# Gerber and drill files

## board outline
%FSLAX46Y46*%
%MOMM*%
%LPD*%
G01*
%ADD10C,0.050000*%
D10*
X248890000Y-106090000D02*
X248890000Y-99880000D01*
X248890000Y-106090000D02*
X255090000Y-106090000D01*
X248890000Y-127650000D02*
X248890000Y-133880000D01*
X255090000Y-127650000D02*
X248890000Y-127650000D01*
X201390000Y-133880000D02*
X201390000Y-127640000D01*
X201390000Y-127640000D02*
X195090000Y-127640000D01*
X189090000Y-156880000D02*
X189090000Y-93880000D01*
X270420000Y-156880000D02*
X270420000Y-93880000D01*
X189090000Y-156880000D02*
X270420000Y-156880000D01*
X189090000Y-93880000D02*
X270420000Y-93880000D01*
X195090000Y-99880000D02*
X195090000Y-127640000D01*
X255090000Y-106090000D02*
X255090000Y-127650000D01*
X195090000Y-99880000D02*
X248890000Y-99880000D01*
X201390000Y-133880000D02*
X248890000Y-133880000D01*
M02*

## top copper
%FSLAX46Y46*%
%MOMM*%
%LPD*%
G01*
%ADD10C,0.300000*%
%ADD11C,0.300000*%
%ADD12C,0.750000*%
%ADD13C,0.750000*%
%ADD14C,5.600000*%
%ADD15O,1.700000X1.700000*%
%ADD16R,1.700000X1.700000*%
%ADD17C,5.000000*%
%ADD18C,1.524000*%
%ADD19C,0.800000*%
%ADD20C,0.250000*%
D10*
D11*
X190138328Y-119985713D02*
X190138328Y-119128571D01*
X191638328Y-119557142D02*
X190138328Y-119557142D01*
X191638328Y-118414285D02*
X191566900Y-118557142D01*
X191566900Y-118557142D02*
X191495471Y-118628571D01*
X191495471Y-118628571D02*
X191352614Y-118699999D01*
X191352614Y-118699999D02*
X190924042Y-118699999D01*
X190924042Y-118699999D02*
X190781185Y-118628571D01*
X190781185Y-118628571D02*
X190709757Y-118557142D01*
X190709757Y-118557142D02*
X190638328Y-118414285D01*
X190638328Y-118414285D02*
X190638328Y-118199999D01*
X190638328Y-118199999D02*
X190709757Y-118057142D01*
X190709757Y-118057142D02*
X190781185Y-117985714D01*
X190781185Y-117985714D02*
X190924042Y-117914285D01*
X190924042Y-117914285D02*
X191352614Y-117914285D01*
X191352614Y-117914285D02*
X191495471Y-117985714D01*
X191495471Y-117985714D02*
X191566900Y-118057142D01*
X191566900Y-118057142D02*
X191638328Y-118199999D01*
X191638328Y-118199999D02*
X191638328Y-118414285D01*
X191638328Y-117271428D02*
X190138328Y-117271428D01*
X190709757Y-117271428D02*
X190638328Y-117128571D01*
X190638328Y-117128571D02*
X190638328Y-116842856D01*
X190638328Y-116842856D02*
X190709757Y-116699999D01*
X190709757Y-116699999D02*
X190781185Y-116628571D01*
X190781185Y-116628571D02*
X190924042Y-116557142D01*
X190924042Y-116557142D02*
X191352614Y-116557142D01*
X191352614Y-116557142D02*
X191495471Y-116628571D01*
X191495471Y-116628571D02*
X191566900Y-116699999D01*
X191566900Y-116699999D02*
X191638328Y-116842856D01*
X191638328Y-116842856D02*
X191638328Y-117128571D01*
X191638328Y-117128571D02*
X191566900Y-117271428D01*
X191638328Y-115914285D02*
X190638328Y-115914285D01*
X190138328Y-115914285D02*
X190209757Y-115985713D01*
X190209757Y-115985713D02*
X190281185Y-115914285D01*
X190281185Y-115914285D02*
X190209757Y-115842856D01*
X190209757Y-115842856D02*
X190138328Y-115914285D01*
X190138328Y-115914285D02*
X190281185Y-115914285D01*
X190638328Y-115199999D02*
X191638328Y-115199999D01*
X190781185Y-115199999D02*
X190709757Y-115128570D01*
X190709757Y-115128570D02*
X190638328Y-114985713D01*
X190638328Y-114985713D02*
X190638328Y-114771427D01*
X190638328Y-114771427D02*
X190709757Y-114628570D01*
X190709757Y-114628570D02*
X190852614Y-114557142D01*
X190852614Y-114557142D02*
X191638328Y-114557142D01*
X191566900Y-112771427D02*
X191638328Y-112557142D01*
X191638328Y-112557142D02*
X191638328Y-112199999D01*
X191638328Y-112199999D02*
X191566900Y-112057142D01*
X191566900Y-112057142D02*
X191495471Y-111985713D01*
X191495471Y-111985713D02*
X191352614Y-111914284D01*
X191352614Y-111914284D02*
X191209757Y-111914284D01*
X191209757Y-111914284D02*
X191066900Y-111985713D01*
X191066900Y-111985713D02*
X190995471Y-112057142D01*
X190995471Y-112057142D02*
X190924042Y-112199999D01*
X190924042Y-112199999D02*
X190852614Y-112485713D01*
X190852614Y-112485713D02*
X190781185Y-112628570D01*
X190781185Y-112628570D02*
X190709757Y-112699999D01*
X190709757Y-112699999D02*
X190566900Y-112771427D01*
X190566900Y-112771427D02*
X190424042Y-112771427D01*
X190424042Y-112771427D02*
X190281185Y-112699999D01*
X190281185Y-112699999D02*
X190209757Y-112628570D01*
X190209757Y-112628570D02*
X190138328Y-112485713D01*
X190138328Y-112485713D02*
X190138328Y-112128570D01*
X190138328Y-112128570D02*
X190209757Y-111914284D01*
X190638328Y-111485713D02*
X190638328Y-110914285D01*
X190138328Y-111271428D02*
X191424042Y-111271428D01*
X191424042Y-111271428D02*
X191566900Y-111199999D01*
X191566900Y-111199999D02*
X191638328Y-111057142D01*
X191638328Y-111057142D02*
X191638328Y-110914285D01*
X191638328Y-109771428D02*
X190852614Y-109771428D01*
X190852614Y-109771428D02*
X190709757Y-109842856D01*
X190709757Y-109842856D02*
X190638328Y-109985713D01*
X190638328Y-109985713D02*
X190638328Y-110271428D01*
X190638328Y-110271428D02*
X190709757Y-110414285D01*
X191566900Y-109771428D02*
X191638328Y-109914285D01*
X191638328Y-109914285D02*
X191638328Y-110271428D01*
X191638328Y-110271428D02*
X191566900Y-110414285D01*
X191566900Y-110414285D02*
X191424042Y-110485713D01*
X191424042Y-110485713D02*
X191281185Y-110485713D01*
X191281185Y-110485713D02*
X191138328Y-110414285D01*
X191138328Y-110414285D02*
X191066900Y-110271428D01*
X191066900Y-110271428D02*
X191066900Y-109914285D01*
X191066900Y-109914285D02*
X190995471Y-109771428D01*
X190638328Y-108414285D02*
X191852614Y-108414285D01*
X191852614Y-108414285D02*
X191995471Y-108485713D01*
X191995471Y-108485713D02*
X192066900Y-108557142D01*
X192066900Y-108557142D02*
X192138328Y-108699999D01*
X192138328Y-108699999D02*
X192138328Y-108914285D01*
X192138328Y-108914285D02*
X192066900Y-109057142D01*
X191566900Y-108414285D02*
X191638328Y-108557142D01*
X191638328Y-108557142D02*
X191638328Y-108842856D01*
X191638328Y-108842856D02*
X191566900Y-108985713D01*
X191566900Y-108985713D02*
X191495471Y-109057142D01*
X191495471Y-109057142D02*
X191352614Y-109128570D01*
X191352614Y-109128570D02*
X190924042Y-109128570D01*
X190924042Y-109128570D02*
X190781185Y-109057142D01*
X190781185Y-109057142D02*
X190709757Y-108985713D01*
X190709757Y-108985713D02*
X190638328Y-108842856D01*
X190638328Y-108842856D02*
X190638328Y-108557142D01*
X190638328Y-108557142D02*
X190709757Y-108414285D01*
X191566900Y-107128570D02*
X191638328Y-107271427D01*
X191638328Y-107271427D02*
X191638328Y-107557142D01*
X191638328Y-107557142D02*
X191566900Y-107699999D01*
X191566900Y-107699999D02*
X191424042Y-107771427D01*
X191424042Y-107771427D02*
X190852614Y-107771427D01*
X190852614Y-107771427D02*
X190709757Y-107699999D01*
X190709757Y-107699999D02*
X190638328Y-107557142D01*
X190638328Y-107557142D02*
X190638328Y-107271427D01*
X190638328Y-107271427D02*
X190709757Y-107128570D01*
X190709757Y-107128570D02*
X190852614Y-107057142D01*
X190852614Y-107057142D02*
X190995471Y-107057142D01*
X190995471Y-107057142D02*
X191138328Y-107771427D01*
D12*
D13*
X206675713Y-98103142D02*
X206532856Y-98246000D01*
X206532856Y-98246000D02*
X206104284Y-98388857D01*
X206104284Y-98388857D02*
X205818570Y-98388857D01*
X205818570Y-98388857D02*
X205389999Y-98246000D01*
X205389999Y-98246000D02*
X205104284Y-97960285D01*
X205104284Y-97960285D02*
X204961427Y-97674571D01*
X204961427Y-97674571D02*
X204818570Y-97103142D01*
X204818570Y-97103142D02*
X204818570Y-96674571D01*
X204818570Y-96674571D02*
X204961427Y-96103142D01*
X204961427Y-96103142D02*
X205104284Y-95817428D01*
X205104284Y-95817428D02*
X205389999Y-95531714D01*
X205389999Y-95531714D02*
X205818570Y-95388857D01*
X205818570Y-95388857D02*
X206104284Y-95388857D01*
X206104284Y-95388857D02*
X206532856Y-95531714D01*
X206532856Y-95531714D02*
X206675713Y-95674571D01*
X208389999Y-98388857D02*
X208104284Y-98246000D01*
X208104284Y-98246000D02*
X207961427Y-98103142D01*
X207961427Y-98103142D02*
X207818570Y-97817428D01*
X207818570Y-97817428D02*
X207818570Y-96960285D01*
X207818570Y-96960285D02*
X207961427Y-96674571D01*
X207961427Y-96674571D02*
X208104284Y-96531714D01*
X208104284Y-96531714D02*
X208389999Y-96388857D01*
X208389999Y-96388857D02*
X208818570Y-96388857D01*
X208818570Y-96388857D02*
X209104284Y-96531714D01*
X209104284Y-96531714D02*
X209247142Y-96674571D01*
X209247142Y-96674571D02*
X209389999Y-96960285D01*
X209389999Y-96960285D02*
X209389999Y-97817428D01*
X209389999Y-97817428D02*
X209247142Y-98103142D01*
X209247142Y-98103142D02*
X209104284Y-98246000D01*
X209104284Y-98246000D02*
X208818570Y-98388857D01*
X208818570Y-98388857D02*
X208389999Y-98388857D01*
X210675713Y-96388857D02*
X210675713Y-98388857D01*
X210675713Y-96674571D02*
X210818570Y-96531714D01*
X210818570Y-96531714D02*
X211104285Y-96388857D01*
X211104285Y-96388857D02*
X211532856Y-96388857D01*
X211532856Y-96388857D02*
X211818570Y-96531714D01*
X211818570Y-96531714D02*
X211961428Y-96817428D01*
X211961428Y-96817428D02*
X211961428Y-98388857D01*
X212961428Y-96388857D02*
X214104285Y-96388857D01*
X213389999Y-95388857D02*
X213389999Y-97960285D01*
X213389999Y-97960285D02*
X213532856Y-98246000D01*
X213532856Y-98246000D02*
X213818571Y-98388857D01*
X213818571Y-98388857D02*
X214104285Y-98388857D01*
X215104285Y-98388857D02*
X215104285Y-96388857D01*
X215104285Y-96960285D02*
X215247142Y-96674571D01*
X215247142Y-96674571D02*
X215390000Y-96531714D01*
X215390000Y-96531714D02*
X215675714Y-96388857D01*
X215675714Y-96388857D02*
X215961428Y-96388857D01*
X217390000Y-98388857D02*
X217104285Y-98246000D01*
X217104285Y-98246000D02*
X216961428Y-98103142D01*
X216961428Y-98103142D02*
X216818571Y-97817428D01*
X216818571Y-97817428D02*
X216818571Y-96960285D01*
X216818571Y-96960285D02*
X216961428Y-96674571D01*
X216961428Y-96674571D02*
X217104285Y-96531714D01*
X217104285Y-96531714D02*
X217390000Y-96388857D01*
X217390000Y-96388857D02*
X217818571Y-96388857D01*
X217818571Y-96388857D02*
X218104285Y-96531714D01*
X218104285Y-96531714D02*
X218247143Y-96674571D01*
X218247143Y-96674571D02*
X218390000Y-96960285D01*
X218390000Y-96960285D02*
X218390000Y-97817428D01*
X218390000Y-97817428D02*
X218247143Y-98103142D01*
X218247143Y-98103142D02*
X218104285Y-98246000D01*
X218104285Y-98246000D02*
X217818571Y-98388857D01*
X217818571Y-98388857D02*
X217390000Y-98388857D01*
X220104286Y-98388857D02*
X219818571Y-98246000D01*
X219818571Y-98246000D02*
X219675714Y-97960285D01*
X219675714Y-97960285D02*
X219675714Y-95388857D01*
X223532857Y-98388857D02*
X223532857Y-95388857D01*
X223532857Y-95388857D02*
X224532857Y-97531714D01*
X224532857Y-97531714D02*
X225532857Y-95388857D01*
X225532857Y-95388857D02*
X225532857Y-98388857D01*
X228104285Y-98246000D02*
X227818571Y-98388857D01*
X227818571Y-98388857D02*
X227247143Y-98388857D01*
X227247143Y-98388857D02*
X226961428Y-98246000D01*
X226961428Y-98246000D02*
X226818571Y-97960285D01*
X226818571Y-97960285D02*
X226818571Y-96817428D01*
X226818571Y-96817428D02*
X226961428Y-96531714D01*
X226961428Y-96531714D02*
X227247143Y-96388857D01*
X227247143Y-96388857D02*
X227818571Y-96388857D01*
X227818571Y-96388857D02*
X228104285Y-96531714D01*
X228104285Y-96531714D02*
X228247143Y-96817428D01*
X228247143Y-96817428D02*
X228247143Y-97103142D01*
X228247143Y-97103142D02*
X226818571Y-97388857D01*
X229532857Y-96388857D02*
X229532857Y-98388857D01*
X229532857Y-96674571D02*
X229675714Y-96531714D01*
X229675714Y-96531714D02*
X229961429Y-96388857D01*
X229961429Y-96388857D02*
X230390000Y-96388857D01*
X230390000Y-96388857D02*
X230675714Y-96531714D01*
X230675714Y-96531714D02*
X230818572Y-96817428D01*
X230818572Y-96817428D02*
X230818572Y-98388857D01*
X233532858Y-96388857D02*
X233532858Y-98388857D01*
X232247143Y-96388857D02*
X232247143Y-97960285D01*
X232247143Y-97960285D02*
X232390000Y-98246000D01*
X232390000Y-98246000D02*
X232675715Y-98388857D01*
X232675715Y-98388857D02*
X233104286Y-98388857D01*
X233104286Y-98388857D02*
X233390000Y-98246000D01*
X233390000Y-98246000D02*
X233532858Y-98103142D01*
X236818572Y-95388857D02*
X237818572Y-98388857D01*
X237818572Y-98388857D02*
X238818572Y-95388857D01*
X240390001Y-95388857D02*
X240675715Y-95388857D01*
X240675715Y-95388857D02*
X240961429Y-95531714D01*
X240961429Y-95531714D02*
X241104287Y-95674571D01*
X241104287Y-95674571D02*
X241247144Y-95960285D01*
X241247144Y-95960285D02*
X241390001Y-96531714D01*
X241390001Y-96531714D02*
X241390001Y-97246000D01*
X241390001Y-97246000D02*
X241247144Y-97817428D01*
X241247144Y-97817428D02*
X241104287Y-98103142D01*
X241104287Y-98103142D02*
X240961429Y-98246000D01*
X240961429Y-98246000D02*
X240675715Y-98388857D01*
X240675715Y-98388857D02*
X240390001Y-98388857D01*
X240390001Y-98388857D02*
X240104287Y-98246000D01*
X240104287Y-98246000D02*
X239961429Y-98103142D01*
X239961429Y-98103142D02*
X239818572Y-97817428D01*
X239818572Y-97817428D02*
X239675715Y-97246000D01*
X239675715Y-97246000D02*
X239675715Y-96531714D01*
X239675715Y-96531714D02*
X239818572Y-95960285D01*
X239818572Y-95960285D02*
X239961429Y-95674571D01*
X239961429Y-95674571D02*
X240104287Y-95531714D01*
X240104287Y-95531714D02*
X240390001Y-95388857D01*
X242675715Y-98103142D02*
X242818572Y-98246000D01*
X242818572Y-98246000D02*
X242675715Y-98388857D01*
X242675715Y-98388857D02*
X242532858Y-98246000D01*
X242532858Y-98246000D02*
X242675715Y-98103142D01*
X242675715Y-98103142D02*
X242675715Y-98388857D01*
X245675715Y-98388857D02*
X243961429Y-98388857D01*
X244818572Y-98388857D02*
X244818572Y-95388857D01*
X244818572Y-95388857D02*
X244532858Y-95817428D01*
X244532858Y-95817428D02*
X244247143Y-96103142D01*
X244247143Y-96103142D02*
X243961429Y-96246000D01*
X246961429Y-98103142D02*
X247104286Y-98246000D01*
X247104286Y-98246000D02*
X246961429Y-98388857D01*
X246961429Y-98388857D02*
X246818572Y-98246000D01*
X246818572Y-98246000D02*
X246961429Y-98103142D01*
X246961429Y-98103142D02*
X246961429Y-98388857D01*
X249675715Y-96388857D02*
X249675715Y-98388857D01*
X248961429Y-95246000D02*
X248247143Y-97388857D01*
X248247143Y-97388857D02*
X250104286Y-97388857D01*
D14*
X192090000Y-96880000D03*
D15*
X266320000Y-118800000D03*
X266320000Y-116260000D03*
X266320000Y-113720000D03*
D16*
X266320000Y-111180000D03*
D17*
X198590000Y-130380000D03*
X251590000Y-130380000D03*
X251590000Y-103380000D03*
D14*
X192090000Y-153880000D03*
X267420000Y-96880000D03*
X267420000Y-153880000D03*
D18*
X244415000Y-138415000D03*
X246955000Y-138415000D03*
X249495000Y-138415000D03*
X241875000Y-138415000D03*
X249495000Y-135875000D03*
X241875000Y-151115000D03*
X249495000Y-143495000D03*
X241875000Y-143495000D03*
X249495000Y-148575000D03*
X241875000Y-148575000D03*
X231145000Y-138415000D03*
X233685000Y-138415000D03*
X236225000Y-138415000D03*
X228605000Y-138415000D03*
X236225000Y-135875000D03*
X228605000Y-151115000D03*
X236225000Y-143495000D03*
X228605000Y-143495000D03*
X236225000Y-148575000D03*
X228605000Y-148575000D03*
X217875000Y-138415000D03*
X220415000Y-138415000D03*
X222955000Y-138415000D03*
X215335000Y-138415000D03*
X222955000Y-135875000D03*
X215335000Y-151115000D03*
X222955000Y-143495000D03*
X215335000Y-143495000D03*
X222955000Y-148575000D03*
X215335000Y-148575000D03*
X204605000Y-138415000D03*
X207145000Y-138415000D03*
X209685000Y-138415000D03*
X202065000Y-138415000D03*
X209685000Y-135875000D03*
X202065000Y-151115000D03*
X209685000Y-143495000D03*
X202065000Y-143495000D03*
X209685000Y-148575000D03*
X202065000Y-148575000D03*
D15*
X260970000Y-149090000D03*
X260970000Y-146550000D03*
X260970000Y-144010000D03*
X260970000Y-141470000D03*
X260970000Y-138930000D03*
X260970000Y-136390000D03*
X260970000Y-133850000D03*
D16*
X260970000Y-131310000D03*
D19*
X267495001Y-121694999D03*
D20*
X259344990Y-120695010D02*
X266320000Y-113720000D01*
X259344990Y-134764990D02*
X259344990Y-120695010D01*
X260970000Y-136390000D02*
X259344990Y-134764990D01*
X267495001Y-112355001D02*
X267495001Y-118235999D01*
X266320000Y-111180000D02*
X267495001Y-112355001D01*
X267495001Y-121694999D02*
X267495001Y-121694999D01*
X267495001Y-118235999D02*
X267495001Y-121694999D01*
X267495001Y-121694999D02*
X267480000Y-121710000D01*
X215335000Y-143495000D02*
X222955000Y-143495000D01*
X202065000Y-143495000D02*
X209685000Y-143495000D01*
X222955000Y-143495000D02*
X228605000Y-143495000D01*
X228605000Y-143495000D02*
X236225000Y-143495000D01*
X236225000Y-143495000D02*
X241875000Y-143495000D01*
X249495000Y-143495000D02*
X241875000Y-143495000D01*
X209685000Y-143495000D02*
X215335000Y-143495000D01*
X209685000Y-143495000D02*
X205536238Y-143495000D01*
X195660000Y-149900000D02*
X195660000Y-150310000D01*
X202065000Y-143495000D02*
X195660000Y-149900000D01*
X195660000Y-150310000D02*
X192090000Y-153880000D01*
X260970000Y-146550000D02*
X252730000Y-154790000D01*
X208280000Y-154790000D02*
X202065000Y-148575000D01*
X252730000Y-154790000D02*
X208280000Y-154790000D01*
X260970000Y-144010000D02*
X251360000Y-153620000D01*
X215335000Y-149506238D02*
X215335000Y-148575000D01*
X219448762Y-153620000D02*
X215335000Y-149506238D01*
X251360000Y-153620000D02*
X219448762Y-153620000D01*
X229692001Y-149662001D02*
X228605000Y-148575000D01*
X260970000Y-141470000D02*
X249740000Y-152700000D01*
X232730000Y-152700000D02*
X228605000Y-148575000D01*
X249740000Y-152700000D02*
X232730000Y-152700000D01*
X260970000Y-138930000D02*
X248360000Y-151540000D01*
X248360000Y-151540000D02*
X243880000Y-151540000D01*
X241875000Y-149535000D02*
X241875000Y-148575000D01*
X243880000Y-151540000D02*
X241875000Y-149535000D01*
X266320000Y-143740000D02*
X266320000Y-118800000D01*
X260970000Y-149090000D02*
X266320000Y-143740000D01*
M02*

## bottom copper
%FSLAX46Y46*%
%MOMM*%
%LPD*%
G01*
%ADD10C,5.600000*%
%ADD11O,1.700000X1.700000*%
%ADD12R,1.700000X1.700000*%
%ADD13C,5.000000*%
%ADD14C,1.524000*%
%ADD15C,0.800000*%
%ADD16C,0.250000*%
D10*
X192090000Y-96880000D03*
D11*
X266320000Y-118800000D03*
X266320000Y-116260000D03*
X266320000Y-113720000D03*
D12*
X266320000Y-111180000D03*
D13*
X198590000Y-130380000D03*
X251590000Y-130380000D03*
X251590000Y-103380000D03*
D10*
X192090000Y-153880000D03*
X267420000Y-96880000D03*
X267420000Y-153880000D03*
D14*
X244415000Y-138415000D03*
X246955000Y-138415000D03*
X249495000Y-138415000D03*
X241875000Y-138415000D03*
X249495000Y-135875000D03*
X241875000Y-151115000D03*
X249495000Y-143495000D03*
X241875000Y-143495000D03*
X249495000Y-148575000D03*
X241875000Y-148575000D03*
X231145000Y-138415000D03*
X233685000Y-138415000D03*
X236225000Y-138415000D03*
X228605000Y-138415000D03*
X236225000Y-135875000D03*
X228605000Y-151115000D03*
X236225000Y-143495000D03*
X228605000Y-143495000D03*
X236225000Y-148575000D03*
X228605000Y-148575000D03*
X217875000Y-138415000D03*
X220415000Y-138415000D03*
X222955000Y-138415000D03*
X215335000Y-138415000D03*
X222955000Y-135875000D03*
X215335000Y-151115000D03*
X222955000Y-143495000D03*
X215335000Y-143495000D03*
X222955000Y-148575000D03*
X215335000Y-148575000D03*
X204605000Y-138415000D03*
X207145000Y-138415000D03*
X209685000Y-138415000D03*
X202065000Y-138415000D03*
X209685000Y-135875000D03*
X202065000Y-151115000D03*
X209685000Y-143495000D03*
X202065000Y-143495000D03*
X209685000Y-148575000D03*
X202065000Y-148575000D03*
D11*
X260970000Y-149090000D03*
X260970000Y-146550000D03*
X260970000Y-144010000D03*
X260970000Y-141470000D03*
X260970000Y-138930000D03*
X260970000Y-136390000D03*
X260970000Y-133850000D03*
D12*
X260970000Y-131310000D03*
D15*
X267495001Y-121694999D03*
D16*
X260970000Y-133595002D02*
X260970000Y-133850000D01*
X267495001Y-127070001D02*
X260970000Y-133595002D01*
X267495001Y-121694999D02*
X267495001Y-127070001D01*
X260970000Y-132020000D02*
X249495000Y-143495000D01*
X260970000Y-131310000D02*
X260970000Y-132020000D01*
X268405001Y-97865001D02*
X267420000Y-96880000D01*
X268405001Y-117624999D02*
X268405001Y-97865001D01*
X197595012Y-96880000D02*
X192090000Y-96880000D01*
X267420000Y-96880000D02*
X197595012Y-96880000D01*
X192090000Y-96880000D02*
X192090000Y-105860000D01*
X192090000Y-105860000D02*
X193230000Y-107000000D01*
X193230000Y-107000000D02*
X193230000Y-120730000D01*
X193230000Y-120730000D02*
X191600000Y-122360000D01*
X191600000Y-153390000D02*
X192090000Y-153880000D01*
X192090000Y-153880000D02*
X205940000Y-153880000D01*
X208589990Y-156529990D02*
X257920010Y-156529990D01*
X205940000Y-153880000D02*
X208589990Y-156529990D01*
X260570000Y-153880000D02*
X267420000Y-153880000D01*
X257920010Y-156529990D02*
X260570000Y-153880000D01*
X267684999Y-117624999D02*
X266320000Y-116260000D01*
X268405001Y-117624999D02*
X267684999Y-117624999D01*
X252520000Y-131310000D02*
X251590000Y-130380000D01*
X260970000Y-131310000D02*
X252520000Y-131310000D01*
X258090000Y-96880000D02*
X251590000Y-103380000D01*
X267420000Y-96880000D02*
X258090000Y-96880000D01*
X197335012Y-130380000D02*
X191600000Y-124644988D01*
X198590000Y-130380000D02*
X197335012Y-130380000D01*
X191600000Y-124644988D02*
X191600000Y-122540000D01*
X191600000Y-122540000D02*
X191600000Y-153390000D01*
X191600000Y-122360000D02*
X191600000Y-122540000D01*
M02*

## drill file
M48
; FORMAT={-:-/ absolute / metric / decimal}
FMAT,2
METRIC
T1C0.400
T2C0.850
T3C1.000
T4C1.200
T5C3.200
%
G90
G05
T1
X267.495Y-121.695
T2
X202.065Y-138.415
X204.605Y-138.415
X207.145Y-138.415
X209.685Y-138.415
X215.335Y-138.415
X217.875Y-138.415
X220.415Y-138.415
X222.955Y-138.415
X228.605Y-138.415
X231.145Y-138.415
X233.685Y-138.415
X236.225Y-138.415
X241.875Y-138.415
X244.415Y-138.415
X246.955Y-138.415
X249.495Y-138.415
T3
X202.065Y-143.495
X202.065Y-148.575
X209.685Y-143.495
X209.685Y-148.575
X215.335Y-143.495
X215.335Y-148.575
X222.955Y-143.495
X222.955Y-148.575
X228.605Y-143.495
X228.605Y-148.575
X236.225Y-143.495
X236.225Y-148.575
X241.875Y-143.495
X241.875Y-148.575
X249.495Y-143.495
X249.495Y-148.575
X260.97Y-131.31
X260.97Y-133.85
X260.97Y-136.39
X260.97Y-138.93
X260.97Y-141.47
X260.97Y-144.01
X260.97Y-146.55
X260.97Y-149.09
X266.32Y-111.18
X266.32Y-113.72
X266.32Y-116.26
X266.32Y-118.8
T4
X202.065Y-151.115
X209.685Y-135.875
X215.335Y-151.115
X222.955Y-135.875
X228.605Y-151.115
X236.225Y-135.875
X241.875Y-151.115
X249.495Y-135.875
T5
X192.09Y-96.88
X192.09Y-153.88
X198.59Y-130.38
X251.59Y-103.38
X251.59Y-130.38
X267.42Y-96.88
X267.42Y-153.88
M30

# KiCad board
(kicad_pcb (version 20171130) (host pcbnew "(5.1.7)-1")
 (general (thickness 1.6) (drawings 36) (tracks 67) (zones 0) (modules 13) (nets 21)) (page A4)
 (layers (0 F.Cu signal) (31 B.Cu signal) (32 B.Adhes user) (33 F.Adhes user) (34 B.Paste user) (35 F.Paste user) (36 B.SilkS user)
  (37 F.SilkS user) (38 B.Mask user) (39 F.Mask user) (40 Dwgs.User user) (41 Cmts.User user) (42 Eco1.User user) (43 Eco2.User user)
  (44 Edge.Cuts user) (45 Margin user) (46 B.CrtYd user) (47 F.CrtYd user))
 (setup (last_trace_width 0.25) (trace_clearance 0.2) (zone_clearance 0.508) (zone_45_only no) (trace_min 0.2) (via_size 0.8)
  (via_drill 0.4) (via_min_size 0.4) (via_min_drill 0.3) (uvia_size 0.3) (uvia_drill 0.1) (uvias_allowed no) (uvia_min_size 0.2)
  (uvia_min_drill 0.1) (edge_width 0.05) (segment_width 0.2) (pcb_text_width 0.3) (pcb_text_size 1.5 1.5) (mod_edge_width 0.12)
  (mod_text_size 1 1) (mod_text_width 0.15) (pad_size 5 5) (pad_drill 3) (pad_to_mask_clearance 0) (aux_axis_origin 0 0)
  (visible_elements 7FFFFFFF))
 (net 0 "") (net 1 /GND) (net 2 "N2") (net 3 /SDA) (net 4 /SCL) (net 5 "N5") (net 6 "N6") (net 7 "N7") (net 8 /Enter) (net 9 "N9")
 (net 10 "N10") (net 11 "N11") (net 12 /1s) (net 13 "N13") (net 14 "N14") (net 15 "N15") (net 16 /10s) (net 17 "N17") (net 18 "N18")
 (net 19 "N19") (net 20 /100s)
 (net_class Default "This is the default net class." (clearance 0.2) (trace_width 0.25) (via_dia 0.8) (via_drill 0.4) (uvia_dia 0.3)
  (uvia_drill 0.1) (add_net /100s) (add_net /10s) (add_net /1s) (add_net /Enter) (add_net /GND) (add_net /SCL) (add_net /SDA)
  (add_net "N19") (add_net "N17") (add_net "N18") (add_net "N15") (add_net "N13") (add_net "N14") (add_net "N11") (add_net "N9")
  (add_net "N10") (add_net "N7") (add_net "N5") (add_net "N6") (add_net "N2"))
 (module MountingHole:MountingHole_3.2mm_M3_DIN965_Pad (layer F.Cu) (at 192.09 96.88)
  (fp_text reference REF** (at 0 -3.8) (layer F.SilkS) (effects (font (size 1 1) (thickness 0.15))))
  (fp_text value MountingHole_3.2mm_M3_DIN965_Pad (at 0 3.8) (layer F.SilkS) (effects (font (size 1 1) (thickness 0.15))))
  (pad 1 thru_hole circle (at 0 0) (size 5.6 5.6) (drill 3.2) (layers *.Cu *.Mask) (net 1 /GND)))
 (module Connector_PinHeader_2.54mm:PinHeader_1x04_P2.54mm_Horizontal (layer B.Cu) (at 266.32 111.18 180)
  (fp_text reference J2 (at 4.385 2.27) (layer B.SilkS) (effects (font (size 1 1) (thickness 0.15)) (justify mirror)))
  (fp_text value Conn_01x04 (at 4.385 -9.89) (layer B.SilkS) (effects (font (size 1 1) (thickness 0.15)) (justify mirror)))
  (pad 4 thru_hole oval (at 0 -7.62 180) (size 1.7 1.7) (drill 1) (layers *.Cu *.Mask) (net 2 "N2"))
  (pad 3 thru_hole oval (at 0 -5.08 180) (size 1.7 1.7) (drill 1) (layers *.Cu *.Mask) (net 1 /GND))
  (pad 2 thru_hole oval (at 0 -2.54 180) (size 1.7 1.7) (drill 1) (layers *.Cu *.Mask) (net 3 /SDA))
  (pad 1 thru_hole rect (at 0 0 180) (size 1.7 1.7) (drill 1) (layers *.Cu *.Mask) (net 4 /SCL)))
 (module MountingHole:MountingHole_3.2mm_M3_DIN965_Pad (layer F.Cu) (at 198.59 130.38)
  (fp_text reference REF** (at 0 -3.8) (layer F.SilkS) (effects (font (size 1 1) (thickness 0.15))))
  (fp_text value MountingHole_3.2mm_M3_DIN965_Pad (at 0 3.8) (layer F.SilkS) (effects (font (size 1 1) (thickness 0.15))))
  (pad 1 thru_hole circle (at 0 0) (size 5 5) (drill 3.2) (layers *.Cu *.Mask) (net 1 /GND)))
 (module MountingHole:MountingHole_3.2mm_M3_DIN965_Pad (layer F.Cu) (at 251.59 130.38)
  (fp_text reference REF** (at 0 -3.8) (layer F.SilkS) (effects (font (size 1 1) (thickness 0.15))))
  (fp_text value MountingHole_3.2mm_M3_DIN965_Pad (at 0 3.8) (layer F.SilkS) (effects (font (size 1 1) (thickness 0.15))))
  (pad 1 thru_hole circle (at 0 0) (size 5 5) (drill 3.2) (layers *.Cu *.Mask) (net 1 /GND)))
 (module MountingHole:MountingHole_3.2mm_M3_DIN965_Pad (layer F.Cu) (at 251.59 103.38)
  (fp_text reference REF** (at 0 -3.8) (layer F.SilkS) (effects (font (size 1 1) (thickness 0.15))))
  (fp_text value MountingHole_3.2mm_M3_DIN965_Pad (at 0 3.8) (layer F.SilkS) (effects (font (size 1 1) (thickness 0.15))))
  (pad 1 thru_hole circle (at 0 0) (size 5 5) (drill 3.2) (layers *.Cu *.Mask) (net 1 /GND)))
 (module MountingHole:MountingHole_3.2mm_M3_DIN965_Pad (layer F.Cu) (at 192.09 153.88)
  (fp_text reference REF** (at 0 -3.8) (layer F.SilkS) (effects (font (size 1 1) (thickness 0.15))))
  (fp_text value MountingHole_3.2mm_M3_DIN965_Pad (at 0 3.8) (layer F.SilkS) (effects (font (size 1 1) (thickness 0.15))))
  (pad 1 thru_hole circle (at 0 0) (size 5.6 5.6) (drill 3.2) (layers *.Cu *.Mask) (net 1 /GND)))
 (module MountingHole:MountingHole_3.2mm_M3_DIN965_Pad (layer F.Cu) (at 267.42 96.88)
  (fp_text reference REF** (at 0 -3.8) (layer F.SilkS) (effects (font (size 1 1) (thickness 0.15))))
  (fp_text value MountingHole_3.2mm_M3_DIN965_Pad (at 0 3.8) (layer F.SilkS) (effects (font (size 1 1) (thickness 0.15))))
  (pad 1 thru_hole circle (at 0 0) (size 5.6 5.6) (drill 3.2) (layers *.Cu *.Mask) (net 1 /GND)))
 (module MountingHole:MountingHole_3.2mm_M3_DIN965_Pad (layer F.Cu) (at 267.42 153.88)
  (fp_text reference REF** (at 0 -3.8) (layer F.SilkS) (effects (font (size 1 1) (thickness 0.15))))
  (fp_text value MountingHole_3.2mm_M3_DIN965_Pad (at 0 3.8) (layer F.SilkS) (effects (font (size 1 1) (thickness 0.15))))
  (pad 1 thru_hole circle (at 0 0) (size 5.6 5.6) (drill 3.2) (layers *.Cu *.Mask) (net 1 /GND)))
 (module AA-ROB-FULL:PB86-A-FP (layer F.Cu) (at 239.515 134.995)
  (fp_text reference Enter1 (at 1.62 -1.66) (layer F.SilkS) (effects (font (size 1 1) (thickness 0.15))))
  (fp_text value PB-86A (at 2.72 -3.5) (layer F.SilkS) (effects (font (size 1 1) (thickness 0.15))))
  (pad 5 thru_hole circle (at 4.9 3.42) (size 1.524 1.524) (drill 0.85) (layers *.Cu *.Mask) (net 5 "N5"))
  (pad 6 thru_hole circle (at 7.44 3.42) (size 1.524 1.524) (drill 0.85) (layers *.Cu *.Mask) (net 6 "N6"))
  (pad 7 thru_hole circle (at 9.98 3.42) (size 1.524 1.524) (drill 0.85) (layers *.Cu *.Mask))
  (pad 4 thru_hole circle (at 2.36 3.42) (size 1.524 1.524) (drill 0.85) (layers *.Cu *.Mask))
  (pad 8 thru_hole circle (at 9.98 0.88) (size 1.524 1.524) (drill 1.2) (layers *.Cu *.Mask))
  (pad 8 thru_hole circle (at 2.36 16.12) (size 1.524 1.524) (drill 1.2) (layers *.Cu *.Mask))
  (pad 1 thru_hole circle (at 9.98 8.5) (size 1.524 1.524) (drill 1) (layers *.Cu *.Mask) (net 1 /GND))
  (pad 1 thru_hole circle (at 2.36 8.5) (size 1.524 1.524) (drill 1) (layers *.Cu *.Mask) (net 1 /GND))
  (pad 3 thru_hole circle (at 9.98 13.58) (size 1.524 1.524) (drill 1) (layers *.Cu *.Mask) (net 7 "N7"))
  (pad 2 thru_hole circle (at 2.36 13.58) (size 1.524 1.524) (drill 1) (layers *.Cu *.Mask) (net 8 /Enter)))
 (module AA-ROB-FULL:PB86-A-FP (layer F.Cu) (at 226.245 134.995)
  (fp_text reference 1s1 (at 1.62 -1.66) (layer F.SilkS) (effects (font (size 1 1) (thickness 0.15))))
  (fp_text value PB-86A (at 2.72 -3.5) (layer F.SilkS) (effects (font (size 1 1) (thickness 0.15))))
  (pad 5 thru_hole circle (at 4.9 3.42) (size 1.524 1.524) (drill 0.85) (layers *.Cu *.Mask) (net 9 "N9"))
  (pad 6 thru_hole circle (at 7.44 3.42) (size 1.524 1.524) (drill 0.85) (layers *.Cu *.Mask) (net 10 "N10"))
  (pad 7 thru_hole circle (at 9.98 3.42) (size 1.524 1.524) (drill 0.85) (layers *.Cu *.Mask))
  (pad 4 thru_hole circle (at 2.36 3.42) (size 1.524 1.524) (drill 0.85) (layers *.Cu *.Mask))
  (pad 8 thru_hole circle (at 9.98 0.88) (size 1.524 1.524) (drill 1.2) (layers *.Cu *.Mask))
  (pad 8 thru_hole circle (at 2.36 16.12) (size 1.524 1.524) (drill 1.2) (layers *.Cu *.Mask))
  (pad 1 thru_hole circle (at 9.98 8.5) (size 1.524 1.524) (drill 1) (layers *.Cu *.Mask) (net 1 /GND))
  (pad 1 thru_hole circle (at 2.36 8.5) (size 1.524 1.524) (drill 1) (layers *.Cu *.Mask) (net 1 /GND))
  (pad 3 thru_hole circle (at 9.98 13.58) (size 1.524 1.524) (drill 1) (layers *.Cu *.Mask) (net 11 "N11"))
  (pad 2 thru_hole circle (at 2.36 13.58) (size 1.524 1.524) (drill 1) (layers *.Cu *.Mask) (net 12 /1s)))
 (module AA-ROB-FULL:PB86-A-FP (layer F.Cu) (at 212.975 134.995)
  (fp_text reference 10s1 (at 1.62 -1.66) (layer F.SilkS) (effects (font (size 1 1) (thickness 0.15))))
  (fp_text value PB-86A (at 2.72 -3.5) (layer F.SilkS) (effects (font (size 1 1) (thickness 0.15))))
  (pad 5 thru_hole circle (at 4.9 3.42) (size 1.524 1.524) (drill 0.85) (layers *.Cu *.Mask) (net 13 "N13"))
  (pad 6 thru_hole circle (at 7.44 3.42) (size 1.524 1.524) (drill 0.85) (layers *.Cu *.Mask) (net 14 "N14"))
  (pad 7 thru_hole circle (at 9.98 3.42) (size 1.524 1.524) (drill 0.85) (layers *.Cu *.Mask))
  (pad 4 thru_hole circle (at 2.36 3.42) (size 1.524 1.524) (drill 0.85) (layers *.Cu *.Mask))
  (pad 8 thru_hole circle (at 9.98 0.88) (size 1.524 1.524) (drill 1.2) (layers *.Cu *.Mask))
  (pad 8 thru_hole circle (at 2.36 16.12) (size 1.524 1.524) (drill 1.2) (layers *.Cu *.Mask))
  (pad 1 thru_hole circle (at 9.98 8.5) (size 1.524 1.524) (drill 1) (layers *.Cu *.Mask) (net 1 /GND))
  (pad 1 thru_hole circle (at 2.36 8.5) (size 1.524 1.524) (drill 1) (layers *.Cu *.Mask) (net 1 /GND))
  (pad 3 thru_hole circle (at 9.98 13.58) (size 1.524 1.524) (drill 1) (layers *.Cu *.Mask) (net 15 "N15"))
  (pad 2 thru_hole circle (at 2.36 13.58) (size 1.524 1.524) (drill 1) (layers *.Cu *.Mask) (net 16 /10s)))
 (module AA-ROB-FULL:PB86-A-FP (layer F.Cu) (at 199.705 134.995)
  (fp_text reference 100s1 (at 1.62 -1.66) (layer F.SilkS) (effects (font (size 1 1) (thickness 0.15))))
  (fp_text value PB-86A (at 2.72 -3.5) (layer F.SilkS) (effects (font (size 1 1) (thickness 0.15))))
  (pad 5 thru_hole circle (at 4.9 3.42) (size 1.524 1.524) (drill 0.85) (layers *.Cu *.Mask) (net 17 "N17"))
  (pad 6 thru_hole circle (at 7.44 3.42) (size 1.524 1.524) (drill 0.85) (layers *.Cu *.Mask) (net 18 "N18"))
  (pad 7 thru_hole circle (at 9.98 3.42) (size 1.524 1.524) (drill 0.85) (layers *.Cu *.Mask))
  (pad 4 thru_hole circle (at 2.36 3.42) (size 1.524 1.524) (drill 0.85) (layers *.Cu *.Mask))
  (pad 8 thru_hole circle (at 9.98 0.88) (size 1.524 1.524) (drill 1.2) (layers *.Cu *.Mask))
  (pad 8 thru_hole circle (at 2.36 16.12) (size 1.524 1.524) (drill 1.2) (layers *.Cu *.Mask))
  (pad 1 thru_hole circle (at 9.98 8.5) (size 1.524 1.524) (drill 1) (layers *.Cu *.Mask) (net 1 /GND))
  (pad 1 thru_hole circle (at 2.36 8.5) (size 1.524 1.524) (drill 1) (layers *.Cu *.Mask) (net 1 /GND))
  (pad 3 thru_hole circle (at 9.98 13.58) (size 1.524 1.524) (drill 1) (layers *.Cu *.Mask) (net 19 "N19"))
  (pad 2 thru_hole circle (at 2.36 13.58) (size 1.524 1.524) (drill 1) (layers *.Cu *.Mask) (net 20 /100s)))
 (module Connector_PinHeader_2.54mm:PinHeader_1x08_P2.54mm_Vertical (layer F.Cu) (at 260.97 131.31)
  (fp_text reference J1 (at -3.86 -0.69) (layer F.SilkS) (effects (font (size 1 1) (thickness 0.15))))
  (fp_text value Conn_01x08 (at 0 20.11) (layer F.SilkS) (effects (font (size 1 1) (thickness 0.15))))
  (pad 8 thru_hole oval (at 0 17.78) (size 1.7 1.7) (drill 1) (layers *.Cu *.Mask) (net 2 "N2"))
  (pad 7 thru_hole oval (at 0 15.24) (size 1.7 1.7) (drill 1) (layers *.Cu *.Mask) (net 20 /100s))
  (pad 6 thru_hole oval (at 0 12.7) (size 1.7 1.7) (drill 1) (layers *.Cu *.Mask) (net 16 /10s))
  (pad 5 thru_hole oval (at 0 10.16) (size 1.7 1.7) (drill 1) (layers *.Cu *.Mask) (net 12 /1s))
  (pad 4 thru_hole oval (at 0 7.62) (size 1.7 1.7) (drill 1) (layers *.Cu *.Mask) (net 8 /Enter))
  (pad 3 thru_hole oval (at 0 5.08) (size 1.7 1.7) (drill 1) (layers *.Cu *.Mask) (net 3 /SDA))
  (pad 2 thru_hole oval (at 0 2.54) (size 1.7 1.7) (drill 1) (layers *.Cu *.Mask) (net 4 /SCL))
  (pad 1 thru_hole rect (at 0 0) (size 1.7 1.7) (drill 1) (layers *.Cu *.Mask) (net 1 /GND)))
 (gr_line (start 248.89 106.09) (end 248.89 99.88) (layer Edge.Cuts) (width 0.05))
 (gr_line (start 248.89 106.09) (end 255.09 106.09) (layer Edge.Cuts) (width 0.05))
 (gr_line (start 248.89 127.65) (end 248.89 133.88) (layer Edge.Cuts) (width 0.05))
 (gr_line (start 255.09 127.65) (end 248.89 127.65) (layer Edge.Cuts) (width 0.05))
 (gr_line (start 201.39 133.88) (end 201.39 127.64) (layer Edge.Cuts) (width 0.05))
 (gr_line (start 201.39 127.64) (end 195.09 127.64) (layer Edge.Cuts) (width 0.05))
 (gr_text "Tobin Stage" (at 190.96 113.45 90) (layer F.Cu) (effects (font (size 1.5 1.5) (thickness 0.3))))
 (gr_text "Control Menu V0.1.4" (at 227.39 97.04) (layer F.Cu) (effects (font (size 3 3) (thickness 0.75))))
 (gr_line (start 189.09 156.88) (end 189.09 93.88) (layer Edge.Cuts) (width 0.05))
 (gr_line (start 270.42 156.88) (end 270.42 93.88) (layer Edge.Cuts) (width 0.05))
 (gr_line (start 189.09 156.88) (end 270.42 156.88) (layer Edge.Cuts) (width 0.05))
 (gr_line (start 189.09 93.88) (end 270.42 93.88) (layer Edge.Cuts) (width 0.05))
 (gr_line (start 195.09 99.88) (end 195.09 127.64) (layer Edge.Cuts) (width 0.05))
 (gr_line (start 255.09 106.09) (end 255.09 127.65) (layer Edge.Cuts) (width 0.05))
 (gr_line (start 195.09 99.88) (end 248.89 99.88) (layer Edge.Cuts) (width 0.05))
 (gr_line (start 201.39 133.88) (end 248.89 133.88) (layer Edge.Cuts) (width 0.05))
 (segment (start 259.34499 120.69501) (end 266.32 113.72) (width 0.25) (layer F.Cu) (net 3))
 (segment (start 259.34499 134.76499) (end 259.34499 120.69501) (width 0.25) (layer F.Cu) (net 3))
 (segment (start 260.97 136.39) (end 259.34499 134.76499) (width 0.25) (layer F.Cu) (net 3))
 (segment (start 267.495001 112.355001) (end 267.495001 118.235999) (width 0.25) (layer F.Cu) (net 4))
 (segment (start 266.32 111.18) (end 267.495001 112.355001) (width 0.25) (layer F.Cu) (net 4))
 (segment (start 267.495001 121.694999) (end 267.495001 121.694999) (width 0.25) (layer F.Cu) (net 4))
 (segment (start 267.495001 118.235999) (end 267.495001 121.694999) (width 0.25) (layer F.Cu) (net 4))
 (segment (start 267.495001 121.694999) (end 267.48 121.71) (width 0.25) (layer F.Cu) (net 4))
 (via (at 267.495001 121.694999) (size 0.8) (drill 0.4) (layers F.Cu B.Cu) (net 4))
 (segment (start 260.97 133.595002) (end 260.97 133.85) (width 0.25) (layer B.Cu) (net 4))
 (segment (start 267.495001 127.070001) (end 260.97 133.595002) (width 0.25) (layer B.Cu) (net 4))
 (segment (start 267.495001 121.694999) (end 267.495001 127.070001) (width 0.25) (layer B.Cu) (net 4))
 (segment (start 215.335 143.495) (end 222.955 143.495) (width 0.25) (layer F.Cu) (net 1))
 (segment (start 202.065 143.495) (end 209.685 143.495) (width 0.25) (layer F.Cu) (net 1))
 (segment (start 222.955 143.495) (end 228.605 143.495) (width 0.25) (layer F.Cu) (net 1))
 (segment (start 228.605 143.495) (end 236.225 143.495) (width 0.25) (layer F.Cu) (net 1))
 (segment (start 236.225 143.495) (end 241.875 143.495) (width 0.25) (layer F.Cu) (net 1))
 (segment (start 249.495 143.495) (end 241.875 143.495) (width 0.25) (layer F.Cu) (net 1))
 (segment (start 260.97 132.02) (end 249.495 143.495) (width 0.25) (layer B.Cu) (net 1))
 (segment (start 260.97 131.31) (end 260.97 132.02) (width 0.25) (layer B.Cu) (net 1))
 (segment (start 268.405001 97.865001) (end 267.42 96.88) (width 0.25) (layer B.Cu) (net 1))
 (segment (start 268.405001 117.624999) (end 268.405001 97.865001) (width 0.25) (layer B.Cu) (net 1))
 (segment (start 197.595012 96.88) (end 192.09 96.88) (width 0.25) (layer B.Cu) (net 1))
 (segment (start 267.42 96.88) (end 197.595012 96.88) (width 0.25) (layer B.Cu) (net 1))
 (segment (start 192.09 96.88) (end 192.09 105.86) (width 0.25) (layer B.Cu) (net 1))
 (segment (start 192.09 105.86) (end 193.23 107) (width 0.25) (layer B.Cu) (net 1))
 (segment (start 193.23 107) (end 193.23 120.73) (width 0.25) (layer B.Cu) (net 1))
 (segment (start 193.23 120.73) (end 191.6 122.36) (width 0.25) (layer B.Cu) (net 1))
 (segment (start 191.6 153.39) (end 192.09 153.88) (width 0.25) (layer B.Cu) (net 1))
 (segment (start 192.09 153.88) (end 205.94 153.88) (width 0.25) (layer B.Cu) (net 1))
 (segment (start 208.58999 156.52999) (end 257.92001 156.52999) (width 0.25) (layer B.Cu) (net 1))
 (segment (start 205.94 153.88) (end 208.58999 156.52999) (width 0.25) (layer B.Cu) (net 1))
 (segment (start 260.57 153.88) (end 267.42 153.88) (width 0.25) (layer B.Cu) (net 1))
 (segment (start 257.92001 156.52999) (end 260.57 153.88) (width 0.25) (layer B.Cu) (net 1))
 (segment (start 267.684999 117.624999) (end 266.32 116.26) (width 0.25) (layer B.Cu) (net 1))
 (segment (start 268.405001 117.624999) (end 267.684999 117.624999) (width 0.25) (layer B.Cu) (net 1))
 (segment (start 252.52 131.31) (end 251.59 130.38) (width 0.25) (layer B.Cu) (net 1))
 (segment (start 260.97 131.31) (end 252.52 131.31) (width 0.25) (layer B.Cu) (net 1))
 (segment (start 258.09 96.88) (end 251.59 103.38) (width 0.25) (layer B.Cu) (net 1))
 (segment (start 267.42 96.88) (end 258.09 96.88) (width 0.25) (layer B.Cu) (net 1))
 (segment (start 197.335012 130.38) (end 191.6 124.644988) (width 0.25) (layer B.Cu) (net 1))
 (segment (start 198.59 130.38) (end 197.335012 130.38) (width 0.25) (layer B.Cu) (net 1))
 (segment (start 191.6 124.644988) (end 191.6 122.54) (width 0.25) (layer B.Cu) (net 1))
 (segment (start 191.6 122.54) (end 191.6 153.39) (width 0.25) (layer B.Cu) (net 1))
 (segment (start 191.6 122.36) (end 191.6 122.54) (width 0.25) (layer B.Cu) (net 1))
 (segment (start 209.685 143.495) (end 215.335 143.495) (width 0.25) (layer F.Cu) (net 1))
 (segment (start 209.685 143.495) (end 205.536238 143.495) (width 0.25) (layer F.Cu) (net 1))
 (segment (start 195.66 149.9) (end 195.66 150.31) (width 0.25) (layer F.Cu) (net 1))
 (segment (start 202.065 143.495) (end 195.66 149.9) (width 0.25) (layer F.Cu) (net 1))
 (segment (start 195.66 150.31) (end 192.09 153.88) (width 0.25) (layer F.Cu) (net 1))
 (segment (start 260.97 146.55) (end 252.73 154.79) (width 0.25) (layer F.Cu) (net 20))
 (segment (start 208.28 154.79) (end 202.065 148.575) (width 0.25) (layer F.Cu) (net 20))
 (segment (start 252.73 154.79) (end 208.28 154.79) (width 0.25) (layer F.Cu) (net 20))
 (segment (start 260.97 144.01) (end 251.36 153.62) (width 0.25) (layer F.Cu) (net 16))
 (segment (start 215.335 149.506238) (end 215.335 148.575) (width 0.25) (layer F.Cu) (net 16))
 (segment (start 219.448762 153.62) (end 215.335 149.506238) (width 0.25) (layer F.Cu) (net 16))
 (segment (start 251.36 153.62) (end 219.448762 153.62) (width 0.25) (layer F.Cu) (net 16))
 (segment (start 229.692001 149.662001) (end 228.605 148.575) (width 0.25) (layer F.Cu) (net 12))
 (segment (start 260.97 141.47) (end 249.74 152.7) (width 0.25) (layer F.Cu) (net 12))
 (segment (start 232.73 152.7) (end 228.605 148.575) (width 0.25) (layer F.Cu) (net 12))
 (segment (start 249.74 152.7) (end 232.73 152.7) (width 0.25) (layer F.Cu) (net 12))
 (segment (start 260.97 138.93) (end 248.36 151.54) (width 0.25) (layer F.Cu) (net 8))
 (segment (start 248.36 151.54) (end 243.88 151.54) (width 0.25) (layer F.Cu) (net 8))
 (segment (start 241.875 149.535) (end 241.875 148.575) (width 0.25) (layer F.Cu) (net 8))
 (segment (start 243.88 151.54) (end 241.875 149.535) (width 0.25) (layer F.Cu) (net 8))
 (segment (start 266.32 143.74) (end 266.32 118.8) (width 0.25) (layer F.Cu) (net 2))
 (segment (start 260.97 149.09) (end 266.32 143.74) (width 0.25) (layer F.Cu) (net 2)))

